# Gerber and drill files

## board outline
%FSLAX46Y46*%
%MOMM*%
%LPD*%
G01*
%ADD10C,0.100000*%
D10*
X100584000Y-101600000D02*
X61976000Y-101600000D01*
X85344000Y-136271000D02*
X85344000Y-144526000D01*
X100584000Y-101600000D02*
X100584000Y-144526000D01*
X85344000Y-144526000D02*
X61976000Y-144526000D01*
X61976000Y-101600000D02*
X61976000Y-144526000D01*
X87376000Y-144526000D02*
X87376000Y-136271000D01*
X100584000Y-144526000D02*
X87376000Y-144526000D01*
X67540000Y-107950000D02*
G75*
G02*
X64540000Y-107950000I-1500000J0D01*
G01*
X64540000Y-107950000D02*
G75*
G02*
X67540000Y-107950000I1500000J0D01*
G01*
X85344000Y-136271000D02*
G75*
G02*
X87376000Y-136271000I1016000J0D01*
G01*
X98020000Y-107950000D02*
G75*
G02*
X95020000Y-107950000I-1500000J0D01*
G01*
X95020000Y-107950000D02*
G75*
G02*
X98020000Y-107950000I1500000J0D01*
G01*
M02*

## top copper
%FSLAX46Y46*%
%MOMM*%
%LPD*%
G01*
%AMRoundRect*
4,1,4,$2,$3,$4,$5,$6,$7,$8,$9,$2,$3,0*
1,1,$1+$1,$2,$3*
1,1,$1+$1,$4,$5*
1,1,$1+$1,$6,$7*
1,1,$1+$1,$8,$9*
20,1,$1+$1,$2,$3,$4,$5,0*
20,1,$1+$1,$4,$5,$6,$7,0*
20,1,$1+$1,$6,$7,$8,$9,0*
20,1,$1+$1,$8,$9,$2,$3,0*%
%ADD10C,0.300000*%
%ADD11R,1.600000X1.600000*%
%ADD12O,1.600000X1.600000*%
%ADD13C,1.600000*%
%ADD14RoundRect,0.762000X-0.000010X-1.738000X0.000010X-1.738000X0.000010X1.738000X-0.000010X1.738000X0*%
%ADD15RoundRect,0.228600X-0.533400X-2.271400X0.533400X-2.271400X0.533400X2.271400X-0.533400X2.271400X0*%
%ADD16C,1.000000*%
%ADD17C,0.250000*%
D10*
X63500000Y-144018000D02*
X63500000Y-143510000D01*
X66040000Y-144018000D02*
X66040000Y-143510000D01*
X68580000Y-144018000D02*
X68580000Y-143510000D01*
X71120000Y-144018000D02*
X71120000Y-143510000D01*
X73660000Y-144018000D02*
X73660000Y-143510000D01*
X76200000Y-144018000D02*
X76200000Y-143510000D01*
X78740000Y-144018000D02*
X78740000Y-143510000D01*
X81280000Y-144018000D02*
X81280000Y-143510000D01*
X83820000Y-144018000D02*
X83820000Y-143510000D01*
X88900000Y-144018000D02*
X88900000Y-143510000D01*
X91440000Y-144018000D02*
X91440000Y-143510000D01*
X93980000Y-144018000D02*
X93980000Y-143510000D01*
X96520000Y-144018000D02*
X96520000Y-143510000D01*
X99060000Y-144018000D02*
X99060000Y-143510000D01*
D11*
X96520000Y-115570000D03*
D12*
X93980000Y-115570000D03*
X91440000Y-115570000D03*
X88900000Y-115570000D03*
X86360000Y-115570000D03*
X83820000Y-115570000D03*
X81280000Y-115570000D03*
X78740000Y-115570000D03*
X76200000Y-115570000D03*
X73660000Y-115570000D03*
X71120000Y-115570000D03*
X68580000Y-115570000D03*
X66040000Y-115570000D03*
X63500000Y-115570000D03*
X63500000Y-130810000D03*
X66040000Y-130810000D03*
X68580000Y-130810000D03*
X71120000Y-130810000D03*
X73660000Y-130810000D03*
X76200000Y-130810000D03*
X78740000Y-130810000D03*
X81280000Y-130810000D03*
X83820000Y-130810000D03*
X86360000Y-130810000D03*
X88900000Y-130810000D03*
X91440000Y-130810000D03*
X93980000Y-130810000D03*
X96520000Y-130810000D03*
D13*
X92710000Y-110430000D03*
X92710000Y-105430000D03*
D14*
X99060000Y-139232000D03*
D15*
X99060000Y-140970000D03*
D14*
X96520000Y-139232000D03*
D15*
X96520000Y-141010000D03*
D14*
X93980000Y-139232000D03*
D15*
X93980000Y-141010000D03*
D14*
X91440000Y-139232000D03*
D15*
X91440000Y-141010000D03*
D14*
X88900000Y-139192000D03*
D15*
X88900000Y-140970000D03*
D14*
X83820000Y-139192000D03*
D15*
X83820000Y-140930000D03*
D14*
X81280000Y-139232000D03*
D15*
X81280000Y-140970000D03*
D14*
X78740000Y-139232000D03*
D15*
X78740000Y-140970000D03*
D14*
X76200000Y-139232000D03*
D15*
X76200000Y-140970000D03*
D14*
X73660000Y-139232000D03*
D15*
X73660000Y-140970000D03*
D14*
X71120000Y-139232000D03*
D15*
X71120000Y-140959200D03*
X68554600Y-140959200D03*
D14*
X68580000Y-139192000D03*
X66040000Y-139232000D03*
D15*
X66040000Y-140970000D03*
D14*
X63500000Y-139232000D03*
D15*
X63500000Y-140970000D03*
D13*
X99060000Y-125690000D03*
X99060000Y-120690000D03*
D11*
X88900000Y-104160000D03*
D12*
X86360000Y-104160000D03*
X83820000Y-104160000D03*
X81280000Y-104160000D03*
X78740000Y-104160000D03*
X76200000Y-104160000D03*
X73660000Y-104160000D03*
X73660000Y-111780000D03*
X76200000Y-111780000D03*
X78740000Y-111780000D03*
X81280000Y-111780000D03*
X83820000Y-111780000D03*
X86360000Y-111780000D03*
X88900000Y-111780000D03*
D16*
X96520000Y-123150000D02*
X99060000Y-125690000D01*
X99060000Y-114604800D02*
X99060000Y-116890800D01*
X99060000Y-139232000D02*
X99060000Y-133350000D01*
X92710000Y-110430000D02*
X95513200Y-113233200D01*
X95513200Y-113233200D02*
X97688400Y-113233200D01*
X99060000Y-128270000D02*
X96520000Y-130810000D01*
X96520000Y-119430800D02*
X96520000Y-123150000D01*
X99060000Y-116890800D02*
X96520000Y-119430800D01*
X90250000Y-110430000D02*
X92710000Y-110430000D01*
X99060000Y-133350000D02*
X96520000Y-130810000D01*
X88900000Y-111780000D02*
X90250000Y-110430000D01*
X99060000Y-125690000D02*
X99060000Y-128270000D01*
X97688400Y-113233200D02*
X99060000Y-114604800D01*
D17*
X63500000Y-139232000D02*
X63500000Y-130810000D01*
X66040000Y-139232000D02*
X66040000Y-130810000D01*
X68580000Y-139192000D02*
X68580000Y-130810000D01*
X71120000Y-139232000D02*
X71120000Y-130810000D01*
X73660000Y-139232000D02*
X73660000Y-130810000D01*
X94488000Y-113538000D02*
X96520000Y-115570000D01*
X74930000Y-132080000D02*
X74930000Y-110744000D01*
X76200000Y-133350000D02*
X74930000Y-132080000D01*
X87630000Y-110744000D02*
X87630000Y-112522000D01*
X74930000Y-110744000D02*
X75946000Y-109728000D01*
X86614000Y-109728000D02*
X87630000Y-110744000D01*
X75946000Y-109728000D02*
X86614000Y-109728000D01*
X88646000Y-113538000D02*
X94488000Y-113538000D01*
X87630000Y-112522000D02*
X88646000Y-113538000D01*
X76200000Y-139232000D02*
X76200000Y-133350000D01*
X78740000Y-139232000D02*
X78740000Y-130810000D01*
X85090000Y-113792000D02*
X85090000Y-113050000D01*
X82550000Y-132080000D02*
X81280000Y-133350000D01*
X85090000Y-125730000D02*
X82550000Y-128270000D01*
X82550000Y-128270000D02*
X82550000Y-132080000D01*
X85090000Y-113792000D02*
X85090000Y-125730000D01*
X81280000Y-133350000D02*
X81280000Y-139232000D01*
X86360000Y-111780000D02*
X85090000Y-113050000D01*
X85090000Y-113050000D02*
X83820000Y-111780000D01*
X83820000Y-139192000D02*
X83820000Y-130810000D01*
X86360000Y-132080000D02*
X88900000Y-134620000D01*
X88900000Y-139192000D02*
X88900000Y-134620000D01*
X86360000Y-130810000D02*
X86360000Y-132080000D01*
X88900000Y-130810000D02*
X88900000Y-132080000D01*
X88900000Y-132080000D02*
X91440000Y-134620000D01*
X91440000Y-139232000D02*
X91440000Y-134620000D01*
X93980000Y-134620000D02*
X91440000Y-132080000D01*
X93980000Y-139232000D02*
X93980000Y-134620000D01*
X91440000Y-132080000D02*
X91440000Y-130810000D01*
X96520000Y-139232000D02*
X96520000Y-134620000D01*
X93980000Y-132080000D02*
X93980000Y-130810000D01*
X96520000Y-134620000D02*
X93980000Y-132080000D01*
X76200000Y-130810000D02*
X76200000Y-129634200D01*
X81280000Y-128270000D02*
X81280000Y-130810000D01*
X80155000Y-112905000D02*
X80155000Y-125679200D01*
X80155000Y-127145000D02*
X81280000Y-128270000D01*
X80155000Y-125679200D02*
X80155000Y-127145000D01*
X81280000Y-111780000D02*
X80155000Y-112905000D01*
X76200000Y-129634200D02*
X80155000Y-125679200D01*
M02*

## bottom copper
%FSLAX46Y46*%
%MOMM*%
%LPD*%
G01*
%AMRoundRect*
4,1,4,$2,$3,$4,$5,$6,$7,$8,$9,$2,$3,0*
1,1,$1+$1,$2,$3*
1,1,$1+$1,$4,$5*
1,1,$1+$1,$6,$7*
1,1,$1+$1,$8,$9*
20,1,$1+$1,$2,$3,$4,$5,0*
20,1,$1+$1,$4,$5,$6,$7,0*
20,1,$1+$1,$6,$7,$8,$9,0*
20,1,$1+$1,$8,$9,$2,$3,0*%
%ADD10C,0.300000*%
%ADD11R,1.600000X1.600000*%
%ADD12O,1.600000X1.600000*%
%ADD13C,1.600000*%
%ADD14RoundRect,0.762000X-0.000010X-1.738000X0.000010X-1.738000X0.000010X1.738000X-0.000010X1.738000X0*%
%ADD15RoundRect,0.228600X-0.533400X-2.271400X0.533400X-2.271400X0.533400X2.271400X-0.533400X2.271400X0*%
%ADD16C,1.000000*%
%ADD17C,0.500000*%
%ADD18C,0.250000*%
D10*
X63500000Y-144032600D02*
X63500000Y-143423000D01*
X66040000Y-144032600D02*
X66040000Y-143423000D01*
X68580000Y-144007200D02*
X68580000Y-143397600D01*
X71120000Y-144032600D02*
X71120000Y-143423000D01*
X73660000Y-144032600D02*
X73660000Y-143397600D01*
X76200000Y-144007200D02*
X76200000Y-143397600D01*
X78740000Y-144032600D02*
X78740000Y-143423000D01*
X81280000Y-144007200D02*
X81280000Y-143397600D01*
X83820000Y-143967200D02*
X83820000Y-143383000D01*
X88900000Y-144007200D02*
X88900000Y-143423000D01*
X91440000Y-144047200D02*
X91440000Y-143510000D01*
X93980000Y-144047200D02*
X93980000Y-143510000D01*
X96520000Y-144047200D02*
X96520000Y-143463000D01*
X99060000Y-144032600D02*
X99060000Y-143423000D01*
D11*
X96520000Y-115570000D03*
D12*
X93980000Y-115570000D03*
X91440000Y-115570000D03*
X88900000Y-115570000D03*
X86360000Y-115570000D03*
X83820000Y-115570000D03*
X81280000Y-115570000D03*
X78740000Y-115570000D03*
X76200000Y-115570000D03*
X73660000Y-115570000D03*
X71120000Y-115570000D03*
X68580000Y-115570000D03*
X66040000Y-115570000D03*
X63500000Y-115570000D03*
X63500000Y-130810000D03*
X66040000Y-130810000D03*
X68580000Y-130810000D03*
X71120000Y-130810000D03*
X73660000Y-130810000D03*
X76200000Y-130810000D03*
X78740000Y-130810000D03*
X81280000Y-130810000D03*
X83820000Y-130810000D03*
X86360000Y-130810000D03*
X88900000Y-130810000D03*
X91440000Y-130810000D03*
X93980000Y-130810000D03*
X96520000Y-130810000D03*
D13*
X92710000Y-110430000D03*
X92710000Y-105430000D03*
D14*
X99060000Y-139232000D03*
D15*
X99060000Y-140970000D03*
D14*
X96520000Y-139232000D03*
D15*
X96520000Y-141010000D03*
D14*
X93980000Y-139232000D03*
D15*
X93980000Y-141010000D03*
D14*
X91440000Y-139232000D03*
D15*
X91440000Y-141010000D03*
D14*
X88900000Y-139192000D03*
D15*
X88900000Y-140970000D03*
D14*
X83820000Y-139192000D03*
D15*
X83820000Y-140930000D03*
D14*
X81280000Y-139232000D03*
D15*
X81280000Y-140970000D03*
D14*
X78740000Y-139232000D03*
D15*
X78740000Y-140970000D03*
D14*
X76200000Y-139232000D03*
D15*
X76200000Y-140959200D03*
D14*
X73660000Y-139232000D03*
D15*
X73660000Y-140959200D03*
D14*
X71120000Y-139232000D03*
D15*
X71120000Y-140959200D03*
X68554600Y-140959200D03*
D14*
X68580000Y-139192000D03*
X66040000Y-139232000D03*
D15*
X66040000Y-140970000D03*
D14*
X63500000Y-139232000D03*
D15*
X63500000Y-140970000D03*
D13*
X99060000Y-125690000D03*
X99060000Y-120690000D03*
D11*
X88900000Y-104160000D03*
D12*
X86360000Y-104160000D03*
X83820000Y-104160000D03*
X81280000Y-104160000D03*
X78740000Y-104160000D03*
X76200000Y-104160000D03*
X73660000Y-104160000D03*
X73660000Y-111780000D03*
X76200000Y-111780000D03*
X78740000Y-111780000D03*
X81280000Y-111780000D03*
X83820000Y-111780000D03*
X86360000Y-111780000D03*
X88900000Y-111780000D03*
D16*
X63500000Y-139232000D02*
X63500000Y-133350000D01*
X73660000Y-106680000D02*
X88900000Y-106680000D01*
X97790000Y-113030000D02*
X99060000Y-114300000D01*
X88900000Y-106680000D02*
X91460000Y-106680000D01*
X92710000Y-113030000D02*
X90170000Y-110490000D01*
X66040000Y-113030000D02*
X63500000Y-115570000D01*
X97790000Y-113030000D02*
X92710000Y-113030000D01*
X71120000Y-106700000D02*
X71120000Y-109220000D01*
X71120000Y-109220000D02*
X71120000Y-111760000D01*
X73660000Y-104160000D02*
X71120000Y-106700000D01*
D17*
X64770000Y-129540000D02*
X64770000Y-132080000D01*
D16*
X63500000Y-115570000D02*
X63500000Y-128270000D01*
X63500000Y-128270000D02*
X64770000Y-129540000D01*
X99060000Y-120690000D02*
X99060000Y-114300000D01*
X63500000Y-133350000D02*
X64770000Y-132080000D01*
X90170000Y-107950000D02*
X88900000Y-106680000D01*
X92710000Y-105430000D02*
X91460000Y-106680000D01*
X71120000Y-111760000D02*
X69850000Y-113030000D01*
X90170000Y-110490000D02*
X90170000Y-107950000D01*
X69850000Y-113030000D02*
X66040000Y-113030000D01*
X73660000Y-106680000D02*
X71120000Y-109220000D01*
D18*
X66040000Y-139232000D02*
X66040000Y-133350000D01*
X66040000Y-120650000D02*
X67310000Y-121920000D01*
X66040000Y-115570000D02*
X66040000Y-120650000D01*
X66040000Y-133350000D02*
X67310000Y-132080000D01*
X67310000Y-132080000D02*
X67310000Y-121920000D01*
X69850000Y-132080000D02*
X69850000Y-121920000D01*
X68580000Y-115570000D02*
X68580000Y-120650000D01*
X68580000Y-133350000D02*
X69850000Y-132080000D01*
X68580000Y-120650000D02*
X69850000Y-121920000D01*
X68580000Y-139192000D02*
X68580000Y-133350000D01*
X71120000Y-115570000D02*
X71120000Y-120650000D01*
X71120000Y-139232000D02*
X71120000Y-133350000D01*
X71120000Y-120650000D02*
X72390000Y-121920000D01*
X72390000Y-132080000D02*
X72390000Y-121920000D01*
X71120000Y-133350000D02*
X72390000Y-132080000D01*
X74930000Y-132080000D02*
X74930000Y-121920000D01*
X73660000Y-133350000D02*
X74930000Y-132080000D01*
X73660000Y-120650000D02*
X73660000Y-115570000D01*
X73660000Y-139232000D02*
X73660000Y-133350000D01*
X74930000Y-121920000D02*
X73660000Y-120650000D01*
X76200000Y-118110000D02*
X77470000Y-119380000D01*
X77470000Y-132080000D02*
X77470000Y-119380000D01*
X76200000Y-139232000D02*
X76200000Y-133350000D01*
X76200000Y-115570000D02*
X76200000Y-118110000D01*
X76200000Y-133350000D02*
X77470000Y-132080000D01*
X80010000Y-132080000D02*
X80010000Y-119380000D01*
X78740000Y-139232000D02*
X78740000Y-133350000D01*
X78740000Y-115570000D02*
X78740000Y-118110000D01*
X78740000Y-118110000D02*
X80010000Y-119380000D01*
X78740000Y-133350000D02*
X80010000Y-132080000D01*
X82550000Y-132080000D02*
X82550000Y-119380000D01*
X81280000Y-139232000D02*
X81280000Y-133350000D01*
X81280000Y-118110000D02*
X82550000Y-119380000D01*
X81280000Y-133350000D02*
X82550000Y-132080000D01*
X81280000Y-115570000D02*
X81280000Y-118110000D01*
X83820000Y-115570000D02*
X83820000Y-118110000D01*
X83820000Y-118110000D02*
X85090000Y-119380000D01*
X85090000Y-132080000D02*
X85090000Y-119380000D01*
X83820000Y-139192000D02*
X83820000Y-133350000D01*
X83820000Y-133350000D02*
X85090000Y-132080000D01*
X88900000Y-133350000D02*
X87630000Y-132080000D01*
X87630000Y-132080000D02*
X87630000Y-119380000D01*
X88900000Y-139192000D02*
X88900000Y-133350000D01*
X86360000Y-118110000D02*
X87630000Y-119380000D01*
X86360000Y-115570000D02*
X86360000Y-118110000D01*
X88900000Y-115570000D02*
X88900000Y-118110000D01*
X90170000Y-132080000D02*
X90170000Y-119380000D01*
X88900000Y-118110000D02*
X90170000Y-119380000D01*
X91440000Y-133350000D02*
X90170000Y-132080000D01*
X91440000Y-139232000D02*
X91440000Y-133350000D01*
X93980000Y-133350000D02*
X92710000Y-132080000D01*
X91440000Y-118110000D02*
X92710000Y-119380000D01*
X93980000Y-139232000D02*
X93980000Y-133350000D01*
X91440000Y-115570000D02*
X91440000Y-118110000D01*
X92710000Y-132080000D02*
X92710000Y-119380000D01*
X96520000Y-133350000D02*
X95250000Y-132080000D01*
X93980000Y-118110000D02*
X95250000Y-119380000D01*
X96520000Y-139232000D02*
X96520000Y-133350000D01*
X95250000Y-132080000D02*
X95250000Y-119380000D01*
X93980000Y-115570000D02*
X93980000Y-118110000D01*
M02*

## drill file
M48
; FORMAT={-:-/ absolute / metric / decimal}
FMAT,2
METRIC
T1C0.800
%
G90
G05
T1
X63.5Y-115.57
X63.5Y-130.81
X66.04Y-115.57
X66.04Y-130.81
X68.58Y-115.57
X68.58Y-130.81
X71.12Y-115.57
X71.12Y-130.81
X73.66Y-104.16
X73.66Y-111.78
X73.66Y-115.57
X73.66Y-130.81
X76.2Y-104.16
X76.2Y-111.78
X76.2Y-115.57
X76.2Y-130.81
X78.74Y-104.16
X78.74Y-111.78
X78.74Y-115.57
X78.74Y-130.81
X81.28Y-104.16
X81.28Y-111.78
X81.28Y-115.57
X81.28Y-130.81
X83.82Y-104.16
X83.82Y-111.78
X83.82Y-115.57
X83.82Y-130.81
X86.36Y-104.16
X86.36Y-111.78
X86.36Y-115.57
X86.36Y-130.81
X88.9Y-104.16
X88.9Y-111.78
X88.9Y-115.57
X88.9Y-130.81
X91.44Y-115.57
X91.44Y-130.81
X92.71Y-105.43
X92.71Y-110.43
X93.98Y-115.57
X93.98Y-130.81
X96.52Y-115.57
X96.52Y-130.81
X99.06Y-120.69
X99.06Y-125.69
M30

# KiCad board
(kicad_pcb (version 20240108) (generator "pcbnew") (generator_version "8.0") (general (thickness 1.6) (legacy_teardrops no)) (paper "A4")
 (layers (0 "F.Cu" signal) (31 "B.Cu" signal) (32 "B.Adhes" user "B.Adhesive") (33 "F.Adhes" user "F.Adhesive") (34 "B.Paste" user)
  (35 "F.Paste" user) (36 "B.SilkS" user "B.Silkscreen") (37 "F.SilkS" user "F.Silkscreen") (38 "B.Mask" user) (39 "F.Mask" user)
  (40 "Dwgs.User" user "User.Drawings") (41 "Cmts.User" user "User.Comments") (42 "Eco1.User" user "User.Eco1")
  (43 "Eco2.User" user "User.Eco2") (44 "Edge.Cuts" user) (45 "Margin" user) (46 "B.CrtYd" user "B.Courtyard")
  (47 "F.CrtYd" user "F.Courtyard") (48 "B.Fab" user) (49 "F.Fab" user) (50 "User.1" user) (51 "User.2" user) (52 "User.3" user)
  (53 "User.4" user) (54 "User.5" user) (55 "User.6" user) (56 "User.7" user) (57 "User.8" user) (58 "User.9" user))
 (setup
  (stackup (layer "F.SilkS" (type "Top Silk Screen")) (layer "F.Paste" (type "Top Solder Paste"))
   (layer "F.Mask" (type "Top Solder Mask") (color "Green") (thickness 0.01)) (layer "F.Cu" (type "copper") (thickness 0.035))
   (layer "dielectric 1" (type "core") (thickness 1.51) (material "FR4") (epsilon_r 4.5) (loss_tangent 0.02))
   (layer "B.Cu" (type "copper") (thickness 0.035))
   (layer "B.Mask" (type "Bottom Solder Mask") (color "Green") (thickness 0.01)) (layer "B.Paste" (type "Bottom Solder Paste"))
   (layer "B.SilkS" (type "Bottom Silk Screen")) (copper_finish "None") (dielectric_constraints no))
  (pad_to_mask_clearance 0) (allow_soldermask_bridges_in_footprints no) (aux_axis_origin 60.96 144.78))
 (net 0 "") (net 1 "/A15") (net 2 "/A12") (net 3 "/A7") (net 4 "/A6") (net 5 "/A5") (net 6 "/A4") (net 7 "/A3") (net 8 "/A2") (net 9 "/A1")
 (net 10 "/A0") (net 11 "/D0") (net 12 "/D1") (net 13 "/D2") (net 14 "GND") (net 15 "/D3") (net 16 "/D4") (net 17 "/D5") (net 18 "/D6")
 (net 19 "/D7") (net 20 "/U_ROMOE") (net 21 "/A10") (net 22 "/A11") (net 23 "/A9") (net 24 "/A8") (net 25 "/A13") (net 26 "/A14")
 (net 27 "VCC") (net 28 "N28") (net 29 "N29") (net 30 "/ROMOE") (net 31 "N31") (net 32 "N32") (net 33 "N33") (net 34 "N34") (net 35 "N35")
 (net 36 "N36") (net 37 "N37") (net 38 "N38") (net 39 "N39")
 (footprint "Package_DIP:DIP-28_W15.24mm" (layer "F.Cu") (at 96.52 115.57 -90)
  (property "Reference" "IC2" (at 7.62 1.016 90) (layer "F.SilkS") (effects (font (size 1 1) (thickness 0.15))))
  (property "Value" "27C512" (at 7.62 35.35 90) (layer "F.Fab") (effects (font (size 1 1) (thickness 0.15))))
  (pad "1" thru_hole rect (at 0 0 270) (size 1.6 1.6) (drill 0.8) (layers "*.Cu" "*.Mask") (remove_unused_layers no) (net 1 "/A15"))
  (pad "2" thru_hole oval (at 0 2.54 270) (size 1.6 1.6) (drill 0.8) (layers "*.Cu" "*.Mask") (remove_unused_layers no) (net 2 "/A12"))
  (pad "3" thru_hole oval (at 0 5.08 270) (size 1.6 1.6) (drill 0.8) (layers "*.Cu" "*.Mask") (remove_unused_layers no) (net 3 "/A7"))
  (pad "4" thru_hole oval (at 0 7.62 270) (size 1.6 1.6) (drill 0.8) (layers "*.Cu" "*.Mask") (remove_unused_layers no) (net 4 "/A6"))
  (pad "5" thru_hole oval (at 0 10.16 270) (size 1.6 1.6) (drill 0.8) (layers "*.Cu" "*.Mask") (remove_unused_layers no) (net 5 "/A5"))
  (pad "6" thru_hole oval (at 0 12.7 270) (size 1.6 1.6) (drill 0.8) (layers "*.Cu" "*.Mask") (remove_unused_layers no) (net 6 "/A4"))
  (pad "7" thru_hole oval (at 0 15.24 270) (size 1.6 1.6) (drill 0.8) (layers "*.Cu" "*.Mask") (remove_unused_layers no) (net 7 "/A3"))
  (pad "8" thru_hole oval (at 0 17.78 270) (size 1.6 1.6) (drill 0.8) (layers "*.Cu" "*.Mask") (remove_unused_layers no) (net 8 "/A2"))
  (pad "9" thru_hole oval (at 0 20.32 270) (size 1.6 1.6) (drill 0.8) (layers "*.Cu" "*.Mask") (remove_unused_layers no) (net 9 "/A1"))
  (pad "10" thru_hole oval (at 0 22.86 270) (size 1.6 1.6) (drill 0.8) (layers "*.Cu" "*.Mask") (remove_unused_layers no) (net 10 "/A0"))
  (pad "11" thru_hole oval (at 0 25.4 270) (size 1.6 1.6) (drill 0.8) (layers "*.Cu" "*.Mask") (remove_unused_layers no) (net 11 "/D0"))
  (pad "12" thru_hole oval (at 0 27.94 270) (size 1.6 1.6) (drill 0.8) (layers "*.Cu" "*.Mask") (remove_unused_layers no) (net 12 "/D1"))
  (pad "13" thru_hole oval (at 0 30.48 270) (size 1.6 1.6) (drill 0.8) (layers "*.Cu" "*.Mask") (remove_unused_layers no) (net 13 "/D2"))
  (pad "14" thru_hole oval (at 0 33.02 270) (size 1.6 1.6) (drill 0.8) (layers "*.Cu" "*.Mask") (remove_unused_layers no) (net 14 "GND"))
  (pad "15" thru_hole oval (at 15.24 33.02 270) (size 1.6 1.6) (drill 0.8) (layers "*.Cu" "*.Mask") (remove_unused_layers no) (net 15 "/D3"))
  (pad "16" thru_hole oval (at 15.24 30.48 270) (size 1.6 1.6) (drill 0.8) (layers "*.Cu" "*.Mask") (remove_unused_layers no) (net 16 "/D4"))
  (pad "17" thru_hole oval (at 15.24 27.94 270) (size 1.6 1.6) (drill 0.8) (layers "*.Cu" "*.Mask") (remove_unused_layers no) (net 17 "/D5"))
  (pad "18" thru_hole oval (at 15.24 25.4 270) (size 1.6 1.6) (drill 0.8) (layers "*.Cu" "*.Mask") (remove_unused_layers no) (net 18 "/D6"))
  (pad "19" thru_hole oval (at 15.24 22.86 270) (size 1.6 1.6) (drill 0.8) (layers "*.Cu" "*.Mask") (remove_unused_layers no) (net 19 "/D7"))
  (pad "20" thru_hole oval (at 15.24 20.32 270) (size 1.6 1.6) (drill 0.8) (layers "*.Cu" "*.Mask") (remove_unused_layers no)
   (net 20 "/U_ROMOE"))
  (pad "21" thru_hole oval (at 15.24 17.78 270) (size 1.6 1.6) (drill 0.8) (layers "*.Cu" "*.Mask") (remove_unused_layers no)
   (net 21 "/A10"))
  (pad "22" thru_hole oval (at 15.24 15.24 270) (size 1.6 1.6) (drill 0.8) (layers "*.Cu" "*.Mask") (remove_unused_layers no)
   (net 20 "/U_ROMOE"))
  (pad "23" thru_hole oval (at 15.24 12.7 270) (size 1.6 1.6) (drill 0.8) (layers "*.Cu" "*.Mask") (remove_unused_layers no) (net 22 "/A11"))
  (pad "24" thru_hole oval (at 15.24 10.16 270) (size 1.6 1.6) (drill 0.8) (layers "*.Cu" "*.Mask") (remove_unused_layers no) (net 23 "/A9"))
  (pad "25" thru_hole oval (at 15.24 7.62 270) (size 1.6 1.6) (drill 0.8) (layers "*.Cu" "*.Mask") (remove_unused_layers no) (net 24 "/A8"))
  (pad "26" thru_hole oval (at 15.24 5.08 270) (size 1.6 1.6) (drill 0.8) (layers "*.Cu" "*.Mask") (remove_unused_layers no) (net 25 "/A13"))
  (pad "27" thru_hole oval (at 15.24 2.54 270) (size 1.6 1.6) (drill 0.8) (layers "*.Cu" "*.Mask") (remove_unused_layers no) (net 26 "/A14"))
  (pad "28" thru_hole oval (at 15.24 0 270) (size 1.6 1.6) (drill 0.8) (layers "*.Cu" "*.Mask") (remove_unused_layers no) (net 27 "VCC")))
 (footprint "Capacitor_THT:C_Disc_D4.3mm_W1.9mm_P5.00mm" (layer "F.Cu") (at 92.71 110.43 90)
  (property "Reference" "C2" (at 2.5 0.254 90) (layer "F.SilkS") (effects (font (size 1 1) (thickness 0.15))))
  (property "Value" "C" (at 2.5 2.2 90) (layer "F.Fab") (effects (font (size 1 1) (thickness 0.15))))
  (pad "1" thru_hole circle (at 0 0 90) (size 1.6 1.6) (drill 0.8) (layers "*.Cu" "*.Mask") (remove_unused_layers no) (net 27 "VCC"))
  (pad "2" thru_hole circle (at 5 0 90) (size 1.6 1.6) (drill 0.8) (layers "*.Cu" "*.Mask") (remove_unused_layers no) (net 14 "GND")))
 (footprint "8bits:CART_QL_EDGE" (layer "F.Cu") (at 73.66 139.994)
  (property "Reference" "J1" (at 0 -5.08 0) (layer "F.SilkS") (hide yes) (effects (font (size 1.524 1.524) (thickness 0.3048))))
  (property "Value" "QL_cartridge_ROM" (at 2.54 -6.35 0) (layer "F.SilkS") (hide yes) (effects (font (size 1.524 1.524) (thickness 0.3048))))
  (fp_line (start -10.16 4.024) (end -10.16 3.516) (stroke (width 0.3) (type solid)) (layer "F.Cu"))
  (fp_line (start -7.62 4.024) (end -7.62 3.516) (stroke (width 0.3) (type solid)) (layer "F.Cu"))
  (fp_line (start -5.08 4.024) (end -5.08 3.516) (stroke (width 0.3) (type solid)) (layer "F.Cu"))
  (fp_line (start -2.54 4.024) (end -2.54 3.516) (stroke (width 0.3) (type solid)) (layer "F.Cu"))
  (fp_line (start 0 4.024) (end 0 3.516) (stroke (width 0.3) (type solid)) (layer "F.Cu"))
  (fp_line (start 2.54 4.024) (end 2.54 3.516) (stroke (width 0.3) (type solid)) (layer "F.Cu"))
  (fp_line (start 5.08 4.024) (end 5.08 3.516) (stroke (width 0.3) (type solid)) (layer "F.Cu"))
  (fp_line (start 7.62 4.024) (end 7.62 3.516) (stroke (width 0.3) (type solid)) (layer "F.Cu"))
  (fp_line (start 10.16 4.024) (end 10.16 3.516) (stroke (width 0.3) (type solid)) (layer "F.Cu"))
  (fp_line (start 15.24 4.024) (end 15.24 3.516) (stroke (width 0.3) (type solid)) (layer "F.Cu"))
  (fp_line (start 17.78 4.024) (end 17.78 3.516) (stroke (width 0.3) (type solid)) (layer "F.Cu"))
  (fp_line (start 20.32 4.024) (end 20.32 3.516) (stroke (width 0.3) (type solid)) (layer "F.Cu"))
  (fp_line (start 22.86 4.024) (end 22.86 3.516) (stroke (width 0.3) (type solid)) (layer "F.Cu"))
  (fp_line (start 25.4 4.024) (end 25.4 3.516) (stroke (width 0.3) (type solid)) (layer "F.Cu"))
  (fp_line (start -10.16 4.0386) (end -10.16 3.429) (stroke (width 0.3) (type solid)) (layer "B.Cu"))
  (fp_line (start -7.62 4.0386) (end -7.62 3.429) (stroke (width 0.3) (type solid)) (layer "B.Cu"))
  (fp_line (start -5.08 4.0132) (end -5.08 3.4036) (stroke (width 0.3) (type solid)) (layer "B.Cu"))
  (fp_line (start -2.54 4.0386) (end -2.54 3.429) (stroke (width 0.3) (type solid)) (layer "B.Cu"))
  (fp_line (start 0 4.0386) (end 0 3.4036) (stroke (width 0.3) (type solid)) (layer "B.Cu"))
  (fp_line (start 2.54 4.0132) (end 2.54 3.4036) (stroke (width 0.3) (type solid)) (layer "B.Cu"))
  (fp_line (start 5.08 4.0386) (end 5.08 3.429) (stroke (width 0.3) (type solid)) (layer "B.Cu"))
  (fp_line (start 7.62 4.0132) (end 7.62 3.4036) (stroke (width 0.3) (type solid)) (layer "B.Cu"))
  (fp_line (start 10.16 3.9732) (end 10.16 3.389) (stroke (width 0.3) (type solid)) (layer "B.Cu"))
  (fp_line (start 15.24 4.0132) (end 15.24 3.429) (stroke (width 0.3) (type solid)) (layer "B.Cu"))
  (fp_line (start 17.78 4.0532) (end 17.78 3.516) (stroke (width 0.3) (type solid)) (layer "B.Cu"))
  (fp_line (start 20.32 4.0532) (end 20.32 3.516) (stroke (width 0.3) (type solid)) (layer "B.Cu"))
  (fp_line (start 22.86 4.0532) (end 22.86 3.469) (stroke (width 0.3) (type solid)) (layer "B.Cu"))
  (fp_line (start 25.4 4.0386) (end 25.4 3.429) (stroke (width 0.3) (type solid)) (layer "B.Cu"))
  (pad "1" connect roundrect (at 25.4 -0.762) (size 1.524 5) (layers "F.Cu") (roundrect_rratio 0.5) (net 27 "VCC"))
  (pad "1" connect roundrect (at 25.4 0.976) (size 1.524 5) (layers "F.Cu") (roundrect_rratio 0.15) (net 27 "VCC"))
  (pad "2" connect roundrect (at 25.4 -0.762) (size 1.524 5) (layers "B.Cu") (roundrect_rratio 0.5) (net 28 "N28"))
  (pad "2" connect roundrect (at 25.4 0.976) (size 1.524 5) (layers "B.Cu") (roundrect_rratio 0.15) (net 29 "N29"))
  (pad "3" connect roundrect (at 22.86 -0.762) (size 1.524 5) (layers "F.Cu") (roundrect_rratio 0.5) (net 26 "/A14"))
  (pad "3" connect roundrect (at 22.86 1.016) (size 1.524 5) (layers "F.Cu") (roundrect_rratio 0.15) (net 26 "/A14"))
  (pad "4" connect roundrect (at 22.86 -0.762) (size 1.524 5) (layers "B.Cu") (roundrect_rratio 0.5) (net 2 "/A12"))
  (pad "4" connect roundrect (at 22.86 1.016) (size 1.524 5) (layers "B.Cu") (roundrect_rratio 0.15) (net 2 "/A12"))
  (pad "5" connect roundrect (at 20.32 -0.762) (size 1.524 5) (layers "F.Cu") (roundrect_rratio 0.5) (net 25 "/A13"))
  (pad "5" connect roundrect (at 20.32 1.016) (size 1.524 5) (layers "F.Cu") (roundrect_rratio 0.15) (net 25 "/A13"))
  (pad "6" connect roundrect (at 20.32 -0.762) (size 1.524 5) (layers "B.Cu") (roundrect_rratio 0.5) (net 3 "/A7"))
  (pad "6" connect roundrect (at 20.32 1.016) (size 1.524 5) (layers "B.Cu") (roundrect_rratio 0.15) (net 3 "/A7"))
  (pad "7" connect roundrect (at 17.78 -0.762) (size 1.524 5) (layers "F.Cu") (roundrect_rratio 0.5) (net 24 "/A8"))
  (pad "7" connect roundrect (at 17.78 1.016) (size 1.524 5) (layers "F.Cu") (roundrect_rratio 0.15) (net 24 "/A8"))
  (pad "8" connect roundrect (at 17.78 -0.762) (size 1.524 5) (layers "B.Cu") (roundrect_rratio 0.5) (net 4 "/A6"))
  (pad "8" connect roundrect (at 17.78 1.016) (size 1.524 5) (layers "B.Cu") (roundrect_rratio 0.15) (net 4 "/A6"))
  (pad "9" connect roundrect (at 15.24 -0.802) (size 1.524 5) (layers "F.Cu") (roundrect_rratio 0.5) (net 23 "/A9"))
  (pad "9" connect roundrect (at 15.24 0.976) (size 1.524 5) (layers "F.Cu") (roundrect_rratio 0.15) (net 23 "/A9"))
  (pad "10" connect roundrect (at 15.24 -0.802) (size 1.524 5) (layers "B.Cu") (roundrect_rratio 0.5) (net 5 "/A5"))
  (pad "10" connect roundrect (at 15.24 0.976) (size 1.524 5) (layers "B.Cu") (roundrect_rratio 0.15) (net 5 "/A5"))
  (pad "11" connect roundrect (at 10.16 -0.802) (size 1.524 5) (layers "F.Cu") (roundrect_rratio 0.5) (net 22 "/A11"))
  (pad "11" connect roundrect (at 10.16 0.936) (size 1.524 5) (layers "F.Cu") (roundrect_rratio 0.15) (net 22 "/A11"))
  (pad "12" connect roundrect (at 10.16 -0.802) (size 1.524 5) (layers "B.Cu") (roundrect_rratio 0.5) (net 6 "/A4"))
  (pad "12" connect roundrect (at 10.16 0.936) (size 1.524 5) (layers "B.Cu") (roundrect_rratio 0.15) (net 6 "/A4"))
  (pad "13" connect roundrect (at 7.62 -0.762) (size 1.524 5) (layers "F.Cu") (roundrect_rratio 0.5) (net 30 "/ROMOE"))
  (pad "13" connect roundrect (at 7.62 0.976) (size 1.524 5) (layers "F.Cu") (roundrect_rratio 0.15) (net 30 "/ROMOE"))
  (pad "14" connect roundrect (at 7.62 -0.762) (size 1.524 5) (layers "B.Cu") (roundrect_rratio 0.5) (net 7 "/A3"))
  (pad "14" connect roundrect (at 7.62 0.976) (size 1.524 5) (layers "B.Cu") (roundrect_rratio 0.15) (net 7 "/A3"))
  (pad "15" connect roundrect (at 5.08 -0.762) (size 1.524 5) (layers "F.Cu") (roundrect_rratio 0.5) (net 21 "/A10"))
  (pad "15" connect roundrect (at 5.08 0.976) (size 1.524 5) (layers "F.Cu") (roundrect_rratio 0.15) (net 21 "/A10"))
  (pad "16" connect roundrect (at 5.08 -0.762) (size 1.524 5) (layers "B.Cu") (roundrect_rratio 0.5) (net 8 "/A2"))
  (pad "16" connect roundrect (at 5.08 0.976) (size 1.524 5) (layers "B.Cu") (roundrect_rratio 0.15) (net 8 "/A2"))
  (pad "17" connect roundrect (at 2.54 -0.762) (size 1.524 5) (layers "F.Cu") (roundrect_rratio 0.5) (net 1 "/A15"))
  (pad "17" connect roundrect (at 2.54 0.976) (size 1.524 5) (layers "F.Cu") (roundrect_rratio 0.15) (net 1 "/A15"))
  (pad "18" connect roundrect (at 2.54 -0.762) (size 1.524 5) (layers "B.Cu") (roundrect_rratio 0.5) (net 9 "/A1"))
  (pad "18" connect roundrect (at 2.54 0.9652) (size 1.524 5) (layers "B.Cu") (roundrect_rratio 0.15) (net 9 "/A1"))
  (pad "19" connect roundrect (at 0 -0.762) (size 1.524 5) (layers "F.Cu") (roundrect_rratio 0.5) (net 19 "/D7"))
  (pad "19" connect roundrect (at 0 0.976) (size 1.524 5) (layers "F.Cu") (roundrect_rratio 0.15) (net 19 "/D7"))
  (pad "20" connect roundrect (at 0 -0.762) (size 1.524 5) (layers "B.Cu") (roundrect_rratio 0.5) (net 10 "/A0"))
  (pad "20" connect roundrect (at 0 0.9652) (size 1.524 5) (layers "B.Cu") (roundrect_rratio 0.15) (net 10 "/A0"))
  (pad "21" connect roundrect (at -2.54 -0.762) (size 1.524 5) (layers "F.Cu") (roundrect_rratio 0.5) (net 18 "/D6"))
  (pad "21" connect roundrect (at -2.54 0.9652) (size 1.524 5) (layers "F.Cu") (roundrect_rratio 0.15) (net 18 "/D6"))
  (pad "22" connect roundrect (at -2.54 -0.762) (size 1.524 5) (layers "B.Cu") (roundrect_rratio 0.5) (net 11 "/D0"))
  (pad "22" connect roundrect (at -2.54 0.9652) (size 1.524 5) (layers "B.Cu") (roundrect_rratio 0.15) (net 11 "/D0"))
  (pad "23" connect roundrect (at -5.1054 0.9652) (size 1.524 5) (layers "F.Cu") (roundrect_rratio 0.15) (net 17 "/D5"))
  (pad "23" connect roundrect (at -5.08 -0.802) (size 1.524 5) (layers "F.Cu") (roundrect_rratio 0.5) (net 17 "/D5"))
  (pad "24" connect roundrect (at -5.1054 0.9652) (size 1.524 5) (layers "B.Cu") (roundrect_rratio 0.15) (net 12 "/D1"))
  (pad "24" connect roundrect (at -5.08 -0.802) (size 1.524 5) (layers "B.Cu") (roundrect_rratio 0.5) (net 12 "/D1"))
  (pad "25" connect roundrect (at -7.62 -0.762) (size 1.524 5) (layers "F.Cu") (roundrect_rratio 0.5) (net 16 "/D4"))
  (pad "25" connect roundrect (at -7.62 0.976) (size 1.524 5) (layers "F.Cu") (roundrect_rratio 0.15) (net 16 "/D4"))
  (pad "26" connect roundrect (at -7.62 -0.762) (size 1.524 5) (layers "B.Cu") (roundrect_rratio 0.5) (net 13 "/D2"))
  (pad "26" connect roundrect (at -7.62 0.976) (size 1.524 5) (layers "B.Cu") (roundrect_rratio 0.15) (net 13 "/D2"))
  (pad "27" connect roundrect (at -10.16 -0.762) (size 1.524 5) (layers "F.Cu") (roundrect_rratio 0.5) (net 15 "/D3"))
  (pad "27" connect roundrect (at -10.16 0.976) (size 1.524 5) (layers "F.Cu") (roundrect_rratio 0.15) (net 15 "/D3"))
  (pad "28" connect roundrect (at -10.16 -0.762) (size 1.524 5) (layers "B.Cu") (roundrect_rratio 0.5) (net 14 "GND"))
  (pad "28" connect roundrect (at -10.16 0.976) (size 1.524 5) (layers "B.Cu") (roundrect_rratio 0.15) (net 14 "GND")))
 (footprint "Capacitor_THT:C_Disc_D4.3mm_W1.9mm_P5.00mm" (layer "F.Cu") (at 99.06 125.69 90)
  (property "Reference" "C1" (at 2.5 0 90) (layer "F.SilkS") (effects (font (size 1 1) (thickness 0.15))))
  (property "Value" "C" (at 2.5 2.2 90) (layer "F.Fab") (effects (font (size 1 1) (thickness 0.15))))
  (pad "1" thru_hole circle (at 0 0 90) (size 1.6 1.6) (drill 0.8) (layers "*.Cu" "*.Mask") (remove_unused_layers no) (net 27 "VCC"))
  (pad "2" thru_hole circle (at 5 0 90) (size 1.6 1.6) (drill 0.8) (layers "*.Cu" "*.Mask") (remove_unused_layers no) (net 14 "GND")))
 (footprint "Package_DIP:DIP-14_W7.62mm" (layer "F.Cu") (at 88.9 104.16 -90)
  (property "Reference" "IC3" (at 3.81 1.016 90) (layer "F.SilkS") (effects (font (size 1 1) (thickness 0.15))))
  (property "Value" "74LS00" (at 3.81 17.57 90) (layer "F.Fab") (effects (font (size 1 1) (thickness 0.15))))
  (pad "1" thru_hole rect (at 0 0 270) (size 1.6 1.6) (drill 0.8) (layers "*.Cu" "*.Mask") (remove_unused_layers no) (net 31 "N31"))
  (pad "2" thru_hole oval (at 0 2.54 270) (size 1.6 1.6) (drill 0.8) (layers "*.Cu" "*.Mask") (remove_unused_layers no) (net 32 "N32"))
  (pad "3" thru_hole oval (at 0 5.08 270) (size 1.6 1.6) (drill 0.8) (layers "*.Cu" "*.Mask") (remove_unused_layers no) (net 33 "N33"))
  (pad "4" thru_hole oval (at 0 7.62 270) (size 1.6 1.6) (drill 0.8) (layers "*.Cu" "*.Mask") (remove_unused_layers no) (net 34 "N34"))
  (pad "5" thru_hole oval (at 0 10.16 270) (size 1.6 1.6) (drill 0.8) (layers "*.Cu" "*.Mask") (remove_unused_layers no) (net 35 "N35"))
  (pad "6" thru_hole oval (at 0 12.7 270) (size 1.6 1.6) (drill 0.8) (layers "*.Cu" "*.Mask") (remove_unused_layers no) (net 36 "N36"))
  (pad "7" thru_hole oval (at 0 15.24 270) (size 1.6 1.6) (drill 0.8) (layers "*.Cu" "*.Mask") (remove_unused_layers no) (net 14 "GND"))
  (pad "8" thru_hole oval (at 7.62 15.24 270) (size 1.6 1.6) (drill 0.8) (layers "*.Cu" "*.Mask") (remove_unused_layers no) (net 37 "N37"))
  (pad "9" thru_hole oval (at 7.62 12.7 270) (size 1.6 1.6) (drill 0.8) (layers "*.Cu" "*.Mask") (remove_unused_layers no) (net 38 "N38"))
  (pad "10" thru_hole oval (at 7.62 10.16 270) (size 1.6 1.6) (drill 0.8) (layers "*.Cu" "*.Mask") (remove_unused_layers no) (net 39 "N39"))
  (pad "11" thru_hole oval (at 7.62 7.62 270) (size 1.6 1.6) (drill 0.8) (layers "*.Cu" "*.Mask") (remove_unused_layers no)
   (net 20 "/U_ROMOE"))
  (pad "12" thru_hole oval (at 7.62 5.08 270) (size 1.6 1.6) (drill 0.8) (layers "*.Cu" "*.Mask") (remove_unused_layers no)
   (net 30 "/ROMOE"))
  (pad "13" thru_hole oval (at 7.62 2.54 270) (size 1.6 1.6) (drill 0.8) (layers "*.Cu" "*.Mask") (remove_unused_layers no)
   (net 30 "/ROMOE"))
  (pad "14" thru_hole oval (at 7.62 0 270) (size 1.6 1.6) (drill 0.8) (layers "*.Cu" "*.Mask") (remove_unused_layers no) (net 27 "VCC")))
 (gr_line (start 100.584 101.6) (end 61.976 101.6) (stroke (width 0.1) (type solid)) (layer "Edge.Cuts"))
 (gr_line (start 85.344 136.271) (end 85.344 144.526) (stroke (width 0.1) (type solid)) (layer "Edge.Cuts"))
 (gr_line (start 100.584 101.6) (end 100.584 144.526) (stroke (width 0.1) (type solid)) (layer "Edge.Cuts"))
 (gr_line (start 85.344 144.526) (end 61.976 144.526) (stroke (width 0.1) (type solid)) (layer "Edge.Cuts"))
 (gr_line (start 61.976 101.6) (end 61.976 144.526) (stroke (width 0.1) (type solid)) (layer "Edge.Cuts"))
 (gr_line (start 87.376 144.526) (end 87.376 136.271) (stroke (width 0.1) (type solid)) (layer "Edge.Cuts"))
 (gr_line (start 100.584 144.526) (end 87.376 144.526) (stroke (width 0.1) (type solid)) (layer "Edge.Cuts"))
 (gr_circle (center 66.04 107.95) (end 67.54 107.95) (stroke (width 0.1) (type default)) (fill none) (layer "Edge.Cuts"))
 (gr_arc (start 85.344 136.271) (mid 86.36 135.255) (end 87.376 136.271) (stroke (width 0.1) (type solid)) (layer "Edge.Cuts"))
 (gr_circle (center 96.52 107.95) (end 98.02 107.95) (stroke (width 0.1) (type default)) (fill none) (layer "Edge.Cuts"))
 (segment (start 96.52 123.15) (end 99.06 125.69) (width 1) (layer "F.Cu") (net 27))
 (segment (start 99.06 114.6048) (end 99.06 116.8908) (width 1) (layer "F.Cu") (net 27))
 (segment (start 99.06 139.232) (end 99.06 133.35) (width 1) (layer "F.Cu") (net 27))
 (segment (start 92.71 110.43) (end 95.5132 113.2332) (width 1) (layer "F.Cu") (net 27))
 (segment (start 95.5132 113.2332) (end 97.6884 113.2332) (width 1) (layer "F.Cu") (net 27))
 (segment (start 99.06 128.27) (end 96.52 130.81) (width 1) (layer "F.Cu") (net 27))
 (segment (start 96.52 119.4308) (end 96.52 123.15) (width 1) (layer "F.Cu") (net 27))
 (segment (start 99.06 116.8908) (end 96.52 119.4308) (width 1) (layer "F.Cu") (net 27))
 (segment (start 90.25 110.43) (end 92.71 110.43) (width 1) (layer "F.Cu") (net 27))
 (segment (start 99.06 133.35) (end 96.52 130.81) (width 1) (layer "F.Cu") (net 27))
 (segment (start 88.9 111.78) (end 90.25 110.43) (width 1) (layer "F.Cu") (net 27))
 (segment (start 99.06 125.69) (end 99.06 128.27) (width 1) (layer "F.Cu") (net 27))
 (segment (start 97.6884 113.2332) (end 99.06 114.6048) (width 1) (layer "F.Cu") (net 27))
 (segment (start 63.5 139.232) (end 63.5 133.35) (width 1) (layer "B.Cu") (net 14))
 (segment (start 73.66 106.68) (end 88.9 106.68) (width 1) (layer "B.Cu") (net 14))
 (segment (start 97.79 113.03) (end 99.06 114.3) (width 1) (layer "B.Cu") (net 14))
 (segment (start 88.9 106.68) (end 91.46 106.68) (width 1) (layer "B.Cu") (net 14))
 (segment (start 92.71 113.03) (end 90.17 110.49) (width 1) (layer "B.Cu") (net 14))
 (segment (start 66.04 113.03) (end 63.5 115.57) (width 1) (layer "B.Cu") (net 14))
 (segment (start 97.79 113.03) (end 92.71 113.03) (width 1) (layer "B.Cu") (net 14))
 (segment (start 71.12 106.7) (end 71.12 109.22) (width 1) (layer "B.Cu") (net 14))
 (segment (start 71.12 109.22) (end 71.12 111.76) (width 1) (layer "B.Cu") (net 14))
 (segment (start 73.66 104.16) (end 71.12 106.7) (width 1) (layer "B.Cu") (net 14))
 (segment (start 64.77 129.54) (end 64.77 132.08) (width 0.5) (layer "B.Cu") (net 14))
 (segment (start 63.5 115.57) (end 63.5 128.27) (width 1) (layer "B.Cu") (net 14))
 (segment (start 63.5 128.27) (end 64.77 129.54) (width 1) (layer "B.Cu") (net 14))
 (segment (start 99.06 120.69) (end 99.06 114.3) (width 1) (layer "B.Cu") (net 14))
 (segment (start 63.5 133.35) (end 64.77 132.08) (width 1) (layer "B.Cu") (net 14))
 (segment (start 90.17 107.95) (end 88.9 106.68) (width 1) (layer "B.Cu") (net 14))
 (segment (start 92.71 105.43) (end 91.46 106.68) (width 1) (layer "B.Cu") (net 14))
 (segment (start 71.12 111.76) (end 69.85 113.03) (width 1) (layer "B.Cu") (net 14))
 (segment (start 90.17 110.49) (end 90.17 107.95) (width 1) (layer "B.Cu") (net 14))
 (segment (start 69.85 113.03) (end 66.04 113.03) (width 1) (layer "B.Cu") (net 14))
 (segment (start 73.66 106.68) (end 71.12 109.22) (width 1) (layer "B.Cu") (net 14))
 (segment (start 63.5 139.232) (end 63.5 130.81) (width 0.25) (layer "F.Cu") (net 15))
 (segment (start 66.04 139.232) (end 66.04 130.81) (width 0.25) (layer "F.Cu") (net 16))
 (segment (start 66.04 139.232) (end 66.04 133.35) (width 0.25) (layer "B.Cu") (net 13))
 (segment (start 66.04 120.65) (end 67.31 121.92) (width 0.25) (layer "B.Cu") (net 13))
 (segment (start 66.04 115.57) (end 66.04 120.65) (width 0.25) (layer "B.Cu") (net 13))
 (segment (start 66.04 133.35) (end 67.31 132.08) (width 0.25) (layer "B.Cu") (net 13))
 (segment (start 67.31 132.08) (end 67.31 121.92) (width 0.25) (layer "B.Cu") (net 13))
 (segment (start 68.58 139.192) (end 68.58 130.81) (width 0.25) (layer "F.Cu") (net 17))
 (segment (start 69.85 132.08) (end 69.85 121.92) (width 0.25) (layer "B.Cu") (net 12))
 (segment (start 68.58 115.57) (end 68.58 120.65) (width 0.25) (layer "B.Cu") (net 12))
 (segment (start 68.58 133.35) (end 69.85 132.08) (width 0.25) (layer "B.Cu") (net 12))
 (segment (start 68.58 120.65) (end 69.85 121.92) (width 0.25) (layer "B.Cu") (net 12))
 (segment (start 68.58 139.192) (end 68.58 133.35) (width 0.25) (layer "B.Cu") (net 12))
 (segment (start 71.12 139.232) (end 71.12 130.81) (width 0.25) (layer "F.Cu") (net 18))
 (segment (start 71.12 115.57) (end 71.12 120.65) (width 0.25) (layer "B.Cu") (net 11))
 (segment (start 71.12 139.232) (end 71.12 133.35) (width 0.25) (layer "B.Cu") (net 11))
 (segment (start 71.12 120.65) (end 72.39 121.92) (width 0.25) (layer "B.Cu") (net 11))
 (segment (start 72.39 132.08) (end 72.39 121.92) (width 0.25) (layer "B.Cu") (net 11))
 (segment (start 71.12 133.35) (end 72.39 132.08) (width 0.25) (layer "B.Cu") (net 11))
 (segment (start 73.66 139.232) (end 73.66 130.81) (width 0.25) (layer "F.Cu") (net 19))
 (segment (start 74.93 132.08) (end 74.93 121.92) (width 0.25) (layer "B.Cu") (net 10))
 (segment (start 73.66 133.35) (end 74.93 132.08) (width 0.25) (layer "B.Cu") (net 10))
 (segment (start 73.66 120.65) (end 73.66 115.57) (width 0.25) (layer "B.Cu") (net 10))
 (segment (start 73.66 139.232) (end 73.66 133.35) (width 0.25) (layer "B.Cu") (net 10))
 (segment (start 74.93 121.92) (end 73.66 120.65) (width 0.25) (layer "B.Cu") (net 10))
 (segment (start 94.488 113.538) (end 96.52 115.57) (width 0.25) (layer "F.Cu") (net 1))
 (segment (start 74.93 132.08) (end 74.93 110.744) (width 0.25) (layer "F.Cu") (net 1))
 (segment (start 76.2 133.35) (end 74.93 132.08) (width 0.25) (layer "F.Cu") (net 1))
 (segment (start 87.63 110.744) (end 87.63 112.522) (width 0.25) (layer "F.Cu") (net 1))
 (segment (start 74.93 110.744) (end 75.946 109.728) (width 0.25) (layer "F.Cu") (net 1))
 (segment (start 86.614 109.728) (end 87.63 110.744) (width 0.25) (layer "F.Cu") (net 1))
 (segment (start 75.946 109.728) (end 86.614 109.728) (width 0.25) (layer "F.Cu") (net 1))
 (segment (start 88.646 113.538) (end 94.488 113.538) (width 0.25) (layer "F.Cu") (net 1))
 (segment (start 87.63 112.522) (end 88.646 113.538) (width 0.25) (layer "F.Cu") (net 1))
 (segment (start 76.2 139.232) (end 76.2 133.35) (width 0.25) (layer "F.Cu") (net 1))
 (segment (start 76.2 118.11) (end 77.47 119.38) (width 0.25) (layer "B.Cu") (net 9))
 (segment (start 77.47 132.08) (end 77.47 119.38) (width 0.25) (layer "B.Cu") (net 9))
 (segment (start 76.2 139.232) (end 76.2 133.35) (width 0.25) (layer "B.Cu") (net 9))
 (segment (start 76.2 115.57) (end 76.2 118.11) (width 0.25) (layer "B.Cu") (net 9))
 (segment (start 76.2 133.35) (end 77.47 132.08) (width 0.25) (layer "B.Cu") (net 9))
 (segment (start 78.74 139.232) (end 78.74 130.81) (width 0.25) (layer "F.Cu") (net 21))
 (segment (start 80.01 132.08) (end 80.01 119.38) (width 0.25) (layer "B.Cu") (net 8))
 (segment (start 78.74 139.232) (end 78.74 133.35) (width 0.25) (layer "B.Cu") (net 8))
 (segment (start 78.74 115.57) (end 78.74 118.11) (width 0.25) (layer "B.Cu") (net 8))
 (segment (start 78.74 118.11) (end 80.01 119.38) (width 0.25) (layer "B.Cu") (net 8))
 (segment (start 78.74 133.35) (end 80.01 132.08) (width 0.25) (layer "B.Cu") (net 8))
 (segment (start 85.09 113.792) (end 85.09 113.05) (width 0.25) (layer "F.Cu") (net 30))
 (segment (start 82.55 132.08) (end 81.28 133.35) (width 0.25) (layer "F.Cu") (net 30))
 (segment (start 85.09 125.73) (end 82.55 128.27) (width 0.25) (layer "F.Cu") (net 30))
 (segment (start 82.55 128.27) (end 82.55 132.08) (width 0.25) (layer "F.Cu") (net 30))
 (segment (start 85.09 113.792) (end 85.09 125.73) (width 0.25) (layer "F.Cu") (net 30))
 (segment (start 81.28 133.35) (end 81.28 139.232) (width 0.25) (layer "F.Cu") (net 30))
 (segment (start 86.36 111.78) (end 85.09 113.05) (width 0.25) (layer "F.Cu") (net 30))
 (segment (start 85.09 113.05) (end 83.82 111.78) (width 0.25) (layer "F.Cu") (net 30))
 (segment (start 82.55 132.08) (end 82.55 119.38) (width 0.25) (layer "B.Cu") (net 7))
 (segment (start 81.28 139.232) (end 81.28 133.35) (width 0.25) (layer "B.Cu") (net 7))
 (segment (start 81.28 118.11) (end 82.55 119.38) (width 0.25) (layer "B.Cu") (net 7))
 (segment (start 81.28 133.35) (end 82.55 132.08) (width 0.25) (layer "B.Cu") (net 7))
 (segment (start 81.28 115.57) (end 81.28 118.11) (width 0.25) (layer "B.Cu") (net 7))
 (segment (start 83.82 139.192) (end 83.82 130.81) (width 0.25) (layer "F.Cu") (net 22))
 (segment (start 83.82 115.57) (end 83.82 118.11) (width 0.25) (layer "B.Cu") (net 6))
 (segment (start 83.82 118.11) (end 85.09 119.38) (width 0.25) (layer "B.Cu") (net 6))
 (segment (start 85.09 132.08) (end 85.09 119.38) (width 0.25) (layer "B.Cu") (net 6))
 (segment (start 83.82 139.192) (end 83.82 133.35) (width 0.25) (layer "B.Cu") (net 6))
 (segment (start 83.82 133.35) (end 85.09 132.08) (width 0.25) (layer "B.Cu") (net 6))
 (segment (start 86.36 132.08) (end 88.9 134.62) (width 0.25) (layer "F.Cu") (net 23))
 (segment (start 88.9 139.192) (end 88.9 134.62) (width 0.25) (layer "F.Cu") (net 23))
 (segment (start 86.36 130.81) (end 86.36 132.08) (width 0.25) (layer "F.Cu") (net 23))
 (segment (start 88.9 133.35) (end 87.63 132.08) (width 0.25) (layer "B.Cu") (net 5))
 (segment (start 87.63 132.08) (end 87.63 119.38) (width 0.25) (layer "B.Cu") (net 5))
 (segment (start 88.9 139.192) (end 88.9 133.35) (width 0.25) (layer "B.Cu") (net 5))
 (segment (start 86.36 118.11) (end 87.63 119.38) (width 0.25) (layer "B.Cu") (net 5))
 (segment (start 86.36 115.57) (end 86.36 118.11) (width 0.25) (layer "B.Cu") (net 5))
 (segment (start 88.9 130.81) (end 88.9 132.08) (width 0.25) (layer "F.Cu") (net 24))
 (segment (start 88.9 132.08) (end 91.44 134.62) (width 0.25) (layer "F.Cu") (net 24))
 (segment (start 91.44 139.232) (end 91.44 134.62) (width 0.25) (layer "F.Cu") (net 24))
 (segment (start 88.9 115.57) (end 88.9 118.11) (width 0.25) (layer "B.Cu") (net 4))
 (segment (start 90.17 132.08) (end 90.17 119.38) (width 0.25) (layer "B.Cu") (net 4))
 (segment (start 88.9 118.11) (end 90.17 119.38) (width 0.25) (layer "B.Cu") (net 4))
 (segment (start 91.44 133.35) (end 90.17 132.08) (width 0.25) (layer "B.Cu") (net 4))
 (segment (start 91.44 139.232) (end 91.44 133.35) (width 0.25) (layer "B.Cu") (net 4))
 (segment (start 93.98 134.62) (end 91.44 132.08) (width 0.25) (layer "F.Cu") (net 25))
 (segment (start 93.98 139.232) (end 93.98 134.62) (width 0.25) (layer "F.Cu") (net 25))
 (segment (start 91.44 132.08) (end 91.44 130.81) (width 0.25) (layer "F.Cu") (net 25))
 (segment (start 93.98 133.35) (end 92.71 132.08) (width 0.25) (layer "B.Cu") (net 3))
 (segment (start 91.44 118.11) (end 92.71 119.38) (width 0.25) (layer "B.Cu") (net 3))
 (segment (start 93.98 139.232) (end 93.98 133.35) (width 0.25) (layer "B.Cu") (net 3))
 (segment (start 91.44 115.57) (end 91.44 118.11) (width 0.25) (layer "B.Cu") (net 3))
 (segment (start 92.71 132.08) (end 92.71 119.38) (width 0.25) (layer "B.Cu") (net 3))
 (segment (start 96.52 139.232) (end 96.52 134.62) (width 0.25) (layer "F.Cu") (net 26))
 (segment (start 93.98 132.08) (end 93.98 130.81) (width 0.25) (layer "F.Cu") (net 26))
 (segment (start 96.52 134.62) (end 93.98 132.08) (width 0.25) (layer "F.Cu") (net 26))
 (segment (start 96.52 133.35) (end 95.25 132.08) (width 0.25) (layer "B.Cu") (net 2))
 (segment (start 93.98 118.11) (end 95.25 119.38) (width 0.25) (layer "B.Cu") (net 2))
 (segment (start 96.52 139.232) (end 96.52 133.35) (width 0.25) (layer "B.Cu") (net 2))
 (segment (start 95.25 132.08) (end 95.25 119.38) (width 0.25) (layer "B.Cu") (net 2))
 (segment (start 93.98 115.57) (end 93.98 118.11) (width 0.25) (layer "B.Cu") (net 2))
 (segment (start 76.2 130.81) (end 76.2 129.6342) (width 0.25) (layer "F.Cu") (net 20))
 (segment (start 81.28 128.27) (end 81.28 130.81) (width 0.25) (layer "F.Cu") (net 20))
 (segment (start 80.155 112.905) (end 80.155 125.6792) (width 0.25) (layer "F.Cu") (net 20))
 (segment (start 80.155 127.145) (end 81.28 128.27) (width 0.25) (layer "F.Cu") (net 20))
 (segment (start 80.155 125.6792) (end 80.155 127.145) (width 0.25) (layer "F.Cu") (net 20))
 (segment (start 81.28 111.78) (end 80.155 112.905) (width 0.25) (layer "F.Cu") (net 20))
 (segment (start 76.2 129.6342) (end 80.155 125.6792) (width 0.25) (layer "F.Cu") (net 20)))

